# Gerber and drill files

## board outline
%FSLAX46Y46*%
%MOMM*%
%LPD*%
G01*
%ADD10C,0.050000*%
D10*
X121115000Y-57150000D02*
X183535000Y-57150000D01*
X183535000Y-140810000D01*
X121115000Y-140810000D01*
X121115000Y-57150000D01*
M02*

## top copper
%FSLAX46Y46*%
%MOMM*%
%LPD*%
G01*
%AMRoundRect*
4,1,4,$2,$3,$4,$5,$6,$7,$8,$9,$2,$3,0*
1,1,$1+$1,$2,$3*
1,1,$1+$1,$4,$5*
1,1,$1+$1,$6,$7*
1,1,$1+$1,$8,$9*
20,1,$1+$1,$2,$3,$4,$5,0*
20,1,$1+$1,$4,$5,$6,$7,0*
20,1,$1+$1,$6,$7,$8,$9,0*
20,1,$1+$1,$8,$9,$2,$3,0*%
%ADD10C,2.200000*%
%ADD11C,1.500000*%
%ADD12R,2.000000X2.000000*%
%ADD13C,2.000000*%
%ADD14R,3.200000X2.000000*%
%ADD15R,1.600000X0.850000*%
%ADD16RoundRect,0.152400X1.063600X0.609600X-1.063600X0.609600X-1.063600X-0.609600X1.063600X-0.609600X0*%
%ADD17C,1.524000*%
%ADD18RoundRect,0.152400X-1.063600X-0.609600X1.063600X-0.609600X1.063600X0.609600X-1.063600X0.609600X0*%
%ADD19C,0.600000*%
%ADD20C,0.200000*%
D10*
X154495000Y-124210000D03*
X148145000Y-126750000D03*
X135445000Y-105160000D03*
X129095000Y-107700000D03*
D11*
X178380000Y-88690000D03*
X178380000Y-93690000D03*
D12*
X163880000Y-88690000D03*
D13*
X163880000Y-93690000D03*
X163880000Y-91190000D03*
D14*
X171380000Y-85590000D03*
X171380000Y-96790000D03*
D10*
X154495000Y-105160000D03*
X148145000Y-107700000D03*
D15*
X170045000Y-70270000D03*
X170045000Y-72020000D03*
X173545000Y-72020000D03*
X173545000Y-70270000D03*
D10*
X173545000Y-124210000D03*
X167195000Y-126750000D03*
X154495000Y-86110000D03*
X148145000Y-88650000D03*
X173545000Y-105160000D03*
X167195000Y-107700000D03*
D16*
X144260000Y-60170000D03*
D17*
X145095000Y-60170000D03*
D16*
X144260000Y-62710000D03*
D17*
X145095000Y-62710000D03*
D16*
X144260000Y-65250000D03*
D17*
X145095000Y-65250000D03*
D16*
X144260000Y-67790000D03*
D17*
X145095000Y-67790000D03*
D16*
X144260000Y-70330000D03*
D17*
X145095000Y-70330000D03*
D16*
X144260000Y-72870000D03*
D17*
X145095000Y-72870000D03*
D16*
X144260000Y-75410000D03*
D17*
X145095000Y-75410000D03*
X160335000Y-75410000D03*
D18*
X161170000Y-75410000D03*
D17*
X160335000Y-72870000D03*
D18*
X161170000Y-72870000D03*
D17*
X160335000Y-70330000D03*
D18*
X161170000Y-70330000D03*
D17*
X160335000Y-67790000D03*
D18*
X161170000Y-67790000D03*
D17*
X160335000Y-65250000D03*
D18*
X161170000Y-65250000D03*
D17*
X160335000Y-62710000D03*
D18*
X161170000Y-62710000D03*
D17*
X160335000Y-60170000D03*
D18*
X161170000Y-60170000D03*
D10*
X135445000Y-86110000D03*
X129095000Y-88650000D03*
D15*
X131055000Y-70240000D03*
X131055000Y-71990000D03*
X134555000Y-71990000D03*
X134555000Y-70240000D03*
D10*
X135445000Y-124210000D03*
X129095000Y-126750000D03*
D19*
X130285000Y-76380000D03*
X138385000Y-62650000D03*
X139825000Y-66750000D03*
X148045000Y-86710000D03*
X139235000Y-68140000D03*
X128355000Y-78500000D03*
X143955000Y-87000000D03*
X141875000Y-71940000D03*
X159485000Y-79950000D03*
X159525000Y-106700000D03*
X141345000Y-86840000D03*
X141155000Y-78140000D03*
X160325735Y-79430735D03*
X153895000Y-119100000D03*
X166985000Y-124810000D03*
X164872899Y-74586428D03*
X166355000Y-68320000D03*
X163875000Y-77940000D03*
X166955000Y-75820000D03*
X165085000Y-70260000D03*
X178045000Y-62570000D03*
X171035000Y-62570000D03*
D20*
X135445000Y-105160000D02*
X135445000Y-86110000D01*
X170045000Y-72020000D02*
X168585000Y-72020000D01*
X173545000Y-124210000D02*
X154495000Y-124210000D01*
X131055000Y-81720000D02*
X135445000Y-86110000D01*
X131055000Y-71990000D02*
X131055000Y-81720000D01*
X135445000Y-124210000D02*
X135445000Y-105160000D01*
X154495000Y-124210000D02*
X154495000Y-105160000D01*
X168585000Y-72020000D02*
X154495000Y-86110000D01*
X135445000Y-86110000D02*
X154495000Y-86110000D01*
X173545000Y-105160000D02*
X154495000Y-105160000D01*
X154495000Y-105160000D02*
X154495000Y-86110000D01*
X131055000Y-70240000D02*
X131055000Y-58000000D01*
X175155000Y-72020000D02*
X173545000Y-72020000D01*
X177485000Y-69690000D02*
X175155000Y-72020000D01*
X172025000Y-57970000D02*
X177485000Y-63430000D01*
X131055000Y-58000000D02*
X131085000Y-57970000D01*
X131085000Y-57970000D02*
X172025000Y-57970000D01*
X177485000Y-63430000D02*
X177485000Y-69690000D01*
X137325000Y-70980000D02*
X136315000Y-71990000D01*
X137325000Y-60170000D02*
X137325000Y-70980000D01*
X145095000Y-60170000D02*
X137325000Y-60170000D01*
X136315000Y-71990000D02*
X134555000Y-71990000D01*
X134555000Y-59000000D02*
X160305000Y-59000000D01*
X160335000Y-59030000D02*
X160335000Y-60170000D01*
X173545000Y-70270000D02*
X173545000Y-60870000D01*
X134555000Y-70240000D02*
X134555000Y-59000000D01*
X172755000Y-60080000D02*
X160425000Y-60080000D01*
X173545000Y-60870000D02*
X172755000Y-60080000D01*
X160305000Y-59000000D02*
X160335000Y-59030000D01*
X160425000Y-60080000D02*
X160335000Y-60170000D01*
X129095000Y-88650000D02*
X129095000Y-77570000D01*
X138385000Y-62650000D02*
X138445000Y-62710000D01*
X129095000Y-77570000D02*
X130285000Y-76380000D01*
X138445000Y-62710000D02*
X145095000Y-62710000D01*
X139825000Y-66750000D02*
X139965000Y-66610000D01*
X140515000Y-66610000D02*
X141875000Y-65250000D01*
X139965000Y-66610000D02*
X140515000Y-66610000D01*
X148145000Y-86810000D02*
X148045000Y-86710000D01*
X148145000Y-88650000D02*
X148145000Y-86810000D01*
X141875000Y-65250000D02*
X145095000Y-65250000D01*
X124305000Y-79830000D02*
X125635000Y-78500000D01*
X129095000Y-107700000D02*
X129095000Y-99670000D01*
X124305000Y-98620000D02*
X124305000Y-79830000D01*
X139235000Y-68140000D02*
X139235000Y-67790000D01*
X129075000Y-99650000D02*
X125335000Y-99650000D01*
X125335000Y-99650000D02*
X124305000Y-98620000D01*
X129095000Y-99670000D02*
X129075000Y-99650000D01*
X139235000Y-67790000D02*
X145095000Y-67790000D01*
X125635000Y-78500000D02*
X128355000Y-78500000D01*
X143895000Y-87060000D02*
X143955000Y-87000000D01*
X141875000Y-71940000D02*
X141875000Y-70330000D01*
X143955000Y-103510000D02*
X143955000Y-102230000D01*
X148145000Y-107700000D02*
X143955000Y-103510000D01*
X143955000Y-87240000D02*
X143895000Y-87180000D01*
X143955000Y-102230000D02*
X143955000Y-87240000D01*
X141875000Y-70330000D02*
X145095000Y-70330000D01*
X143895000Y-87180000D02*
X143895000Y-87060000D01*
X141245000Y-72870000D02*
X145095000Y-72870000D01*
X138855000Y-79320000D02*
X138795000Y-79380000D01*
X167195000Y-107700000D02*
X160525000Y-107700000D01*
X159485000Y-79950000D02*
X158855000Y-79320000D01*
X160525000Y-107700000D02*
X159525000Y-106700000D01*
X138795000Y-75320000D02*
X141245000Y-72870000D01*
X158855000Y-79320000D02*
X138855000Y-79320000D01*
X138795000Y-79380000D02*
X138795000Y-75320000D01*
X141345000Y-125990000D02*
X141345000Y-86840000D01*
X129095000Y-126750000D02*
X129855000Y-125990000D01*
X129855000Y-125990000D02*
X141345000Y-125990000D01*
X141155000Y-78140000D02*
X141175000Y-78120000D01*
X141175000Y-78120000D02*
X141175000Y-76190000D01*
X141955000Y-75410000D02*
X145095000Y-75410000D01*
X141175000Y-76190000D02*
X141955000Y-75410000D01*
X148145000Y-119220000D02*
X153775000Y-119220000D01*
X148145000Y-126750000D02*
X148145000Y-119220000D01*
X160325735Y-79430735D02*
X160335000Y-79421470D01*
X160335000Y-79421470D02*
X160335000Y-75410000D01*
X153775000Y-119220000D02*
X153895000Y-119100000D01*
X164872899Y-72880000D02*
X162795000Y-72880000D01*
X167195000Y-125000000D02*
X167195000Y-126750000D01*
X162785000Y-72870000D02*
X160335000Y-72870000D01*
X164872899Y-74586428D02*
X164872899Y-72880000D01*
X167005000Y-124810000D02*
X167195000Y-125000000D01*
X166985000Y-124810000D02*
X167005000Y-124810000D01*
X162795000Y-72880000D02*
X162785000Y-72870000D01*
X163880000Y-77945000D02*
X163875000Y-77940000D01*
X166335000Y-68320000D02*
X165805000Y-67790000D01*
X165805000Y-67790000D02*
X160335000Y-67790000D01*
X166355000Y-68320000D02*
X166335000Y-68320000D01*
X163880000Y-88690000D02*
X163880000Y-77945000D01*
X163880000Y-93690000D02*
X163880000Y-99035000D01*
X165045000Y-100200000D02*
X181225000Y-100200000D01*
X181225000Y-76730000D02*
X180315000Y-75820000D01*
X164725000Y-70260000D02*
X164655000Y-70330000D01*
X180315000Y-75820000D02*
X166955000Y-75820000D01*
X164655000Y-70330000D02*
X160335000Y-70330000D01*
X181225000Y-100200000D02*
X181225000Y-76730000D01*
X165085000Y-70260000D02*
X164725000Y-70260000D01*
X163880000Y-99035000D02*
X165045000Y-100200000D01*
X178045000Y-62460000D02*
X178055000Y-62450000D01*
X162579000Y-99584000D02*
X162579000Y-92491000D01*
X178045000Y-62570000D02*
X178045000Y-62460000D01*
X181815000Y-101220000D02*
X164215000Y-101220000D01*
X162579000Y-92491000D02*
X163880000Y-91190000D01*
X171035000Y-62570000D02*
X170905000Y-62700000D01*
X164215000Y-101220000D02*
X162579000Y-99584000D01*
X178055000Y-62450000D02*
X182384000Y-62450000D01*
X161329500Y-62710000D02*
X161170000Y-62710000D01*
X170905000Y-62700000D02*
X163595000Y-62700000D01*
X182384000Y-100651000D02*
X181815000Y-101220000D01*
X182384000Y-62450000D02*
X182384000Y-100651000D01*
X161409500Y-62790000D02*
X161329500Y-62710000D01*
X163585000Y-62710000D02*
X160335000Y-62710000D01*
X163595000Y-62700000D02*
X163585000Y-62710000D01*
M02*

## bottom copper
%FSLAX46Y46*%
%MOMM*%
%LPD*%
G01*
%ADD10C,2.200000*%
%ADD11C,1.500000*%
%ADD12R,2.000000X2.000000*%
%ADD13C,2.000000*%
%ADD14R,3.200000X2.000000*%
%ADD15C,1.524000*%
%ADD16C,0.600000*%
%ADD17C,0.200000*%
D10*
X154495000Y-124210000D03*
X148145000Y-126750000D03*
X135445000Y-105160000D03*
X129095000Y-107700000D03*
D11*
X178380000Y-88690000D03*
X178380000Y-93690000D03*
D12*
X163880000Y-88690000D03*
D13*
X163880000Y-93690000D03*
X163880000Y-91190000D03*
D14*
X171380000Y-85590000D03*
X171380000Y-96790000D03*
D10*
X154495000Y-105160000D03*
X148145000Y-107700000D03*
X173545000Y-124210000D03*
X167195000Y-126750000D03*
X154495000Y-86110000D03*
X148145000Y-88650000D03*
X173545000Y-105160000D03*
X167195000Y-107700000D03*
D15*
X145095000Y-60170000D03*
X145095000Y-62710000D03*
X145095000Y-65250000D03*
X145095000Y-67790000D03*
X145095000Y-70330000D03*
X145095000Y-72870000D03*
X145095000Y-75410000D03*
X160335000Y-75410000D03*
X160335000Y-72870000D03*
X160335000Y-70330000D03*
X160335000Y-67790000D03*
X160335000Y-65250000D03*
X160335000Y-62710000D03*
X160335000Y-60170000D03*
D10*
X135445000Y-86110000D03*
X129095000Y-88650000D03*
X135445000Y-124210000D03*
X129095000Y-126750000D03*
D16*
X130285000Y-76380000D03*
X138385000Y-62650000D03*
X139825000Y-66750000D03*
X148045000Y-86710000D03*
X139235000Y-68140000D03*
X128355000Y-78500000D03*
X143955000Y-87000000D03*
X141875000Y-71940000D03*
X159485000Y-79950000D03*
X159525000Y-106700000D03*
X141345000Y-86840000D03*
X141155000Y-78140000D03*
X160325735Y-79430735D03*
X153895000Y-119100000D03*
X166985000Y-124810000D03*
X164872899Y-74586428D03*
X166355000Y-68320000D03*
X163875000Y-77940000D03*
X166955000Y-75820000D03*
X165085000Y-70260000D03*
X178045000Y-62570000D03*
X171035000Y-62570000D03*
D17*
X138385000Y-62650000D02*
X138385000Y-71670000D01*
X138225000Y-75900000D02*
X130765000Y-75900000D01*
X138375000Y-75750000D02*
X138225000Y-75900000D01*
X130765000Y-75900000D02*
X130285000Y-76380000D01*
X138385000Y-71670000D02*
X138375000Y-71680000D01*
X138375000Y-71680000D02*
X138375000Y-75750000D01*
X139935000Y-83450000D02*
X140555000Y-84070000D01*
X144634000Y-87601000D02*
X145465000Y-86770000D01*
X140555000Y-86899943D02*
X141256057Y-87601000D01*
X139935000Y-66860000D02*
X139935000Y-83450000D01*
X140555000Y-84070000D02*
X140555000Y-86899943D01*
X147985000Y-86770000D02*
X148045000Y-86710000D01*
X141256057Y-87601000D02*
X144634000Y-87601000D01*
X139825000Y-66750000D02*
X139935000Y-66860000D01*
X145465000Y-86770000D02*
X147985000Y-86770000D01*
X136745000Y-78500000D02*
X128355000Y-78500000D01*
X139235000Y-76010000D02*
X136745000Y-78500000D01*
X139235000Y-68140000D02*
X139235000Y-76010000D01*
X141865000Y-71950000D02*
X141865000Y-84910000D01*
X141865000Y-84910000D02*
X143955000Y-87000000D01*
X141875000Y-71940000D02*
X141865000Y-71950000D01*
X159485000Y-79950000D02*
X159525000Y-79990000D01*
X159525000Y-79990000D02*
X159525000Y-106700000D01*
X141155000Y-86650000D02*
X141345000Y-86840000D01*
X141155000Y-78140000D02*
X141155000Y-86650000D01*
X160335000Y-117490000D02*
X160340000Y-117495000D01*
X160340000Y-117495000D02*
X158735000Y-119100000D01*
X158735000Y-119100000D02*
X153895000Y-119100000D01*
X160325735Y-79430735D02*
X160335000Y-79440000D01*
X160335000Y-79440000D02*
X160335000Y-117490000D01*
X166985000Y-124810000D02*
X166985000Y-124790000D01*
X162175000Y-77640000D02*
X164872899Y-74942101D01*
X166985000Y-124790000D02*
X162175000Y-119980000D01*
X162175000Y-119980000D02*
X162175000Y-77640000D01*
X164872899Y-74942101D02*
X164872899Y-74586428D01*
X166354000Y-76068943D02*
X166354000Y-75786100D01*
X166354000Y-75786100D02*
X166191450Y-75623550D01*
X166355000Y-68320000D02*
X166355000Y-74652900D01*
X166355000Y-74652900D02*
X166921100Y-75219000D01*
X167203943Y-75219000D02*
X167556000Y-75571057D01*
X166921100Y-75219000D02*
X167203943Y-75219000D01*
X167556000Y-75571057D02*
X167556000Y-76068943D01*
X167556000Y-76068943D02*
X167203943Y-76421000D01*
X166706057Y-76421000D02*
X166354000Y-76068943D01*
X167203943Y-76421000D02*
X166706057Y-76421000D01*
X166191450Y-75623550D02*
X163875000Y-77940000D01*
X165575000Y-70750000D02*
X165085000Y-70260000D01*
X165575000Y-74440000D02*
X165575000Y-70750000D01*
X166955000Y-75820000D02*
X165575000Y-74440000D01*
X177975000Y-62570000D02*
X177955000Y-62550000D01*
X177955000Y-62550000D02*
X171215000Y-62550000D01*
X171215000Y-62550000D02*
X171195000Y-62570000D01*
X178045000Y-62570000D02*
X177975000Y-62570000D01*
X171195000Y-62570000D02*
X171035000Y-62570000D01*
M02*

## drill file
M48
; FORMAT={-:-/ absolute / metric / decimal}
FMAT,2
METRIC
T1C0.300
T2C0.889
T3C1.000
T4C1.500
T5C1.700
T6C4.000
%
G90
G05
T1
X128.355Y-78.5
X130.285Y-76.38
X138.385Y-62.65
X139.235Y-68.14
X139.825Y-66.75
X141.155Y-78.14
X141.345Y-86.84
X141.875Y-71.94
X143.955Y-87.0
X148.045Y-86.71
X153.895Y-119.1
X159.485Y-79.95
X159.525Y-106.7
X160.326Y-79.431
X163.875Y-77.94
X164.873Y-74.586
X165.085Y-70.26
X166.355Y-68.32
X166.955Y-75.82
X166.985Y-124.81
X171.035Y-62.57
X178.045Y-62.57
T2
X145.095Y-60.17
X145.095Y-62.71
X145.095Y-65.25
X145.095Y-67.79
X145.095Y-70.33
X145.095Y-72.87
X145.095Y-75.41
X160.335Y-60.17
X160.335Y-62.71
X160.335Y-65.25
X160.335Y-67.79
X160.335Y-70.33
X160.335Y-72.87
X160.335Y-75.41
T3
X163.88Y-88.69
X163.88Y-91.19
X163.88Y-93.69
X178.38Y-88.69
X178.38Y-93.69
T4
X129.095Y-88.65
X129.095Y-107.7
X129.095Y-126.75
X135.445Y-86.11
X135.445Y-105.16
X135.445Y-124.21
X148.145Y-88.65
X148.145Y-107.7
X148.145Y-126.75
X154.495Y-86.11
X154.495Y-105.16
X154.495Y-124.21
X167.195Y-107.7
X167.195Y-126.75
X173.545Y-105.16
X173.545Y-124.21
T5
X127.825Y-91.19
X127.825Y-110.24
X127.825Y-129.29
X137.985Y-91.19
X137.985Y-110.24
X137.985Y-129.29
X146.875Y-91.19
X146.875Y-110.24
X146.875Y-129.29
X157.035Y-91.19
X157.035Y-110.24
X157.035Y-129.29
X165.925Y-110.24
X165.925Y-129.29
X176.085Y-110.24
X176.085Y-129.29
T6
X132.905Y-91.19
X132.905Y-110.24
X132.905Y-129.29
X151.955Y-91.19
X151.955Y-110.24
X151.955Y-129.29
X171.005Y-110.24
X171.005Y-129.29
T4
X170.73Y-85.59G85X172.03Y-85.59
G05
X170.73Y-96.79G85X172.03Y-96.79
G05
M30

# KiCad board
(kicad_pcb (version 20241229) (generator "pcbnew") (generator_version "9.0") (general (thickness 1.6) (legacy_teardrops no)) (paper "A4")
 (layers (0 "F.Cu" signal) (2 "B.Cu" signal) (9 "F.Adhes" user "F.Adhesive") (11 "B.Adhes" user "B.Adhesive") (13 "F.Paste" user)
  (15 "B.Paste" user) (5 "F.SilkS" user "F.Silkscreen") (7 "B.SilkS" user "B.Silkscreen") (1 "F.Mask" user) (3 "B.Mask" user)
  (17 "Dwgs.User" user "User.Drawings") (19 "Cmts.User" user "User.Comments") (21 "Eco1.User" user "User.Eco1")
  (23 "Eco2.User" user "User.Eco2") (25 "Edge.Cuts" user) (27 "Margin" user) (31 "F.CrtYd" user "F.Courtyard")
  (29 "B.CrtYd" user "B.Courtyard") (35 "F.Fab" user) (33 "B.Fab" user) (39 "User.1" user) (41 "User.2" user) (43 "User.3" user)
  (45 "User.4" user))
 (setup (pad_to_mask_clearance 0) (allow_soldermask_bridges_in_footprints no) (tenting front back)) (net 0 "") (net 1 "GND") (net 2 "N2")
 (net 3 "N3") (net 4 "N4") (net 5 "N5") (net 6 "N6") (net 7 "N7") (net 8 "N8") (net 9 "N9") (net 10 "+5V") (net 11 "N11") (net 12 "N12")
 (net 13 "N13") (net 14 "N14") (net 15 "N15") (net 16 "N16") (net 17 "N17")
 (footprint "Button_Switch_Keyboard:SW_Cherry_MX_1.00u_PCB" (layer "F.Cu") (at 154.495 124.21)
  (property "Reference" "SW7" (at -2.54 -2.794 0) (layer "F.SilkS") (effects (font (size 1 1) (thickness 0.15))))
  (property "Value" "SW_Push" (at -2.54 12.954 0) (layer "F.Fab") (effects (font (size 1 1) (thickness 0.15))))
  (pad "" np_thru_hole circle (at -7.62 5.08) (size 1.7 1.7) (drill 1.7) (layers "*.Cu" "*.Mask"))
  (pad "" np_thru_hole circle (at -2.54 5.08) (size 4 4) (drill 4) (layers "*.Cu" "*.Mask"))
  (pad "" np_thru_hole circle (at 2.54 5.08) (size 1.7 1.7) (drill 1.7) (layers "*.Cu" "*.Mask"))
  (pad "1" thru_hole circle (at 0 0) (size 2.2 2.2) (drill 1.5) (layers "*.Cu" "*.Mask") (remove_unused_layers no) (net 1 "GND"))
  (pad "2" thru_hole circle (at -6.35 2.54) (size 2.2 2.2) (drill 1.5) (layers "*.Cu" "*.Mask") (remove_unused_layers no) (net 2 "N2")))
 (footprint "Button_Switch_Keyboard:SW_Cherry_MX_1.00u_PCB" (layer "F.Cu") (at 135.445 105.16)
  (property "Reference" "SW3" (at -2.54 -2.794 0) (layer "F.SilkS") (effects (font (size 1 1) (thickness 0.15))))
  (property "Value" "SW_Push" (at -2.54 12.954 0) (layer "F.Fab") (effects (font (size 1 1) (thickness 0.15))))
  (pad "" np_thru_hole circle (at -7.62 5.08) (size 1.7 1.7) (drill 1.7) (layers "*.Cu" "*.Mask"))
  (pad "" np_thru_hole circle (at -2.54 5.08) (size 4 4) (drill 4) (layers "*.Cu" "*.Mask"))
  (pad "" np_thru_hole circle (at 2.54 5.08) (size 1.7 1.7) (drill 1.7) (layers "*.Cu" "*.Mask"))
  (pad "1" thru_hole circle (at 0 0) (size 2.2 2.2) (drill 1.5) (layers "*.Cu" "*.Mask") (remove_unused_layers no) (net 1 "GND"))
  (pad "2" thru_hole circle (at -6.35 2.54) (size 2.2 2.2) (drill 1.5) (layers "*.Cu" "*.Mask") (remove_unused_layers no) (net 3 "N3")))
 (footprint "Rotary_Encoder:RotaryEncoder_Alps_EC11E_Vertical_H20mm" (layer "F.Cu") (at 163.88 88.69)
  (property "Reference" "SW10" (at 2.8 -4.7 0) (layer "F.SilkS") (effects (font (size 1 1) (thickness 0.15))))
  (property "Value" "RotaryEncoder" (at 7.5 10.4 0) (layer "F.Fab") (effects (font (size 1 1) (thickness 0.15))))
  (pad "" thru_hole circle (at 14.5 0) (size 1.5 1.5) (drill 1) (layers "*.Cu" "*.Mask") (remove_unused_layers no))
  (pad "" thru_hole circle (at 14.5 5) (size 1.5 1.5) (drill 1) (layers "*.Cu" "*.Mask") (remove_unused_layers no))
  (pad "A" thru_hole rect (at 0 0) (size 2 2) (drill 1) (layers "*.Cu" "*.Mask") (remove_unused_layers no) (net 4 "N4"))
  (pad "B" thru_hole circle (at 0 5) (size 2 2) (drill 1) (layers "*.Cu" "*.Mask") (remove_unused_layers no) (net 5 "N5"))
  (pad "C" thru_hole circle (at 0 2.5) (size 2 2) (drill 1) (layers "*.Cu" "*.Mask") (remove_unused_layers no) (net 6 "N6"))
  (pad "MP" thru_hole rect (at 7.5 -3.1) (size 3.2 2) (drill oval 2.8 1.5) (layers "*.Cu" "*.Mask") (remove_unused_layers no))
  (pad "MP" thru_hole rect (at 7.5 8.1) (size 3.2 2) (drill oval 2.8 1.5) (layers "*.Cu" "*.Mask") (remove_unused_layers no)))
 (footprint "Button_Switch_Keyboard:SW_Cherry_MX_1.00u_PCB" (layer "F.Cu") (at 154.495 105.16)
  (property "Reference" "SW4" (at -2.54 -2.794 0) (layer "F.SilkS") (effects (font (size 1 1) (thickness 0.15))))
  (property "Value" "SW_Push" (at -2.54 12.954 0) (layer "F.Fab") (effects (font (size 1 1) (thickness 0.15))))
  (pad "" np_thru_hole circle (at -7.62 5.08) (size 1.7 1.7) (drill 1.7) (layers "*.Cu" "*.Mask"))
  (pad "" np_thru_hole circle (at -2.54 5.08) (size 4 4) (drill 4) (layers "*.Cu" "*.Mask"))
  (pad "" np_thru_hole circle (at 2.54 5.08) (size 1.7 1.7) (drill 1.7) (layers "*.Cu" "*.Mask"))
  (pad "1" thru_hole circle (at 0 0) (size 2.2 2.2) (drill 1.5) (layers "*.Cu" "*.Mask") (remove_unused_layers no) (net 1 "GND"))
  (pad "2" thru_hole circle (at -6.35 2.54) (size 2.2 2.2) (drill 1.5) (layers "*.Cu" "*.Mask") (remove_unused_layers no) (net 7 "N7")))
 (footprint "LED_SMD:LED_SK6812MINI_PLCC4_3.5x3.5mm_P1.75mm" (layer "F.Cu") (at 171.795 71.145)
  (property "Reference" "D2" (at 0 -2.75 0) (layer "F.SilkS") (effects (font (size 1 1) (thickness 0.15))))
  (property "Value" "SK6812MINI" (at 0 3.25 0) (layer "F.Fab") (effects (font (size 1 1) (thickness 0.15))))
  (pad "1" smd rect (at -1.75 -0.875) (size 1.6 0.85) (layers "F.Cu" "F.Mask" "F.Paste") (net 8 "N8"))
  (pad "2" smd rect (at -1.75 0.875) (size 1.6 0.85) (layers "F.Cu" "F.Mask" "F.Paste") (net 1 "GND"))
  (pad "3" smd rect (at 1.75 0.875) (size 1.6 0.85) (layers "F.Cu" "F.Mask" "F.Paste") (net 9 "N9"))
  (pad "4" smd rect (at 1.75 -0.875) (size 1.6 0.85) (layers "F.Cu" "F.Mask" "F.Paste") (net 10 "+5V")))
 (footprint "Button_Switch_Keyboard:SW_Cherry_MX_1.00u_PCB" (layer "F.Cu") (at 173.545 124.21)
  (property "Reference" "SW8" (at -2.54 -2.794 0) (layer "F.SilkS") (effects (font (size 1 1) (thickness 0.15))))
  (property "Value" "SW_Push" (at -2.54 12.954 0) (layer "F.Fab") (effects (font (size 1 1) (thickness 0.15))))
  (pad "" np_thru_hole circle (at -7.62 5.08) (size 1.7 1.7) (drill 1.7) (layers "*.Cu" "*.Mask"))
  (pad "" np_thru_hole circle (at -2.54 5.08) (size 4 4) (drill 4) (layers "*.Cu" "*.Mask"))
  (pad "" np_thru_hole circle (at 2.54 5.08) (size 1.7 1.7) (drill 1.7) (layers "*.Cu" "*.Mask"))
  (pad "1" thru_hole circle (at 0 0) (size 2.2 2.2) (drill 1.5) (layers "*.Cu" "*.Mask") (remove_unused_layers no) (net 1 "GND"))
  (pad "2" thru_hole circle (at -6.35 2.54) (size 2.2 2.2) (drill 1.5) (layers "*.Cu" "*.Mask") (remove_unused_layers no) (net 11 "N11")))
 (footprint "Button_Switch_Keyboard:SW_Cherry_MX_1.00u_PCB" (layer "F.Cu") (at 154.495 86.11)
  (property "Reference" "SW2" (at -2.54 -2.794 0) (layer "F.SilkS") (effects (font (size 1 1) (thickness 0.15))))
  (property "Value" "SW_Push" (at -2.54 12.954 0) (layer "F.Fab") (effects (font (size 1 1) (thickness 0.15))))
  (pad "" np_thru_hole circle (at -7.62 5.08) (size 1.7 1.7) (drill 1.7) (layers "*.Cu" "*.Mask"))
  (pad "" np_thru_hole circle (at -2.54 5.08) (size 4 4) (drill 4) (layers "*.Cu" "*.Mask"))
  (pad "" np_thru_hole circle (at 2.54 5.08) (size 1.7 1.7) (drill 1.7) (layers "*.Cu" "*.Mask"))
  (pad "1" thru_hole circle (at 0 0) (size 2.2 2.2) (drill 1.5) (layers "*.Cu" "*.Mask") (remove_unused_layers no) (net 1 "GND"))
  (pad "2" thru_hole circle (at -6.35 2.54) (size 2.2 2.2) (drill 1.5) (layers "*.Cu" "*.Mask") (remove_unused_layers no) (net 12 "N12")))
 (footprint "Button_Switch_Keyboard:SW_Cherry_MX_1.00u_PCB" (layer "F.Cu") (at 173.545 105.16)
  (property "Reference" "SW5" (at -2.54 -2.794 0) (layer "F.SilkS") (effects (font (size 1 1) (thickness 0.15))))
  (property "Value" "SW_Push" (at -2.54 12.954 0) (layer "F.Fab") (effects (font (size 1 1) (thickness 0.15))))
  (pad "" np_thru_hole circle (at -7.62 5.08) (size 1.7 1.7) (drill 1.7) (layers "*.Cu" "*.Mask"))
  (pad "" np_thru_hole circle (at -2.54 5.08) (size 4 4) (drill 4) (layers "*.Cu" "*.Mask"))
  (pad "" np_thru_hole circle (at 2.54 5.08) (size 1.7 1.7) (drill 1.7) (layers "*.Cu" "*.Mask"))
  (pad "1" thru_hole circle (at 0 0) (size 2.2 2.2) (drill 1.5) (layers "*.Cu" "*.Mask") (remove_unused_layers no) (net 1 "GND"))
  (pad "2" thru_hole circle (at -6.35 2.54) (size 2.2 2.2) (drill 1.5) (layers "*.Cu" "*.Mask") (remove_unused_layers no) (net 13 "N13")))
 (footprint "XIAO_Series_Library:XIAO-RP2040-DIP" (layer "F.Cu") (at 152.715 67.79)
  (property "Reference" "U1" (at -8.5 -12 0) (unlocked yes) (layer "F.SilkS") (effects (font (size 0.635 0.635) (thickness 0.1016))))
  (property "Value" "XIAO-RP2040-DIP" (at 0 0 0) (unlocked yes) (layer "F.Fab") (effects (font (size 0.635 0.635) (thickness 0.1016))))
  (pad "1" smd roundrect (at -8.455 -7.62 180) (size 2.432 1.524) (layers "F.Cu" "F.Mask") (roundrect_rratio 0.1) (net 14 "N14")
   (thermal_bridge_angle 45))
  (pad "1" thru_hole circle (at -7.62 -7.62 180) (size 1.524 1.524) (drill 0.889) (layers "*.Cu" "*.Mask") (remove_unused_layers no)
   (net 14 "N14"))
  (pad "2" smd roundrect (at -8.455 -5.08 180) (size 2.432 1.524) (layers "F.Cu" "F.Mask") (roundrect_rratio 0.1) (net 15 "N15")
   (thermal_bridge_angle 45))
  (pad "2" thru_hole circle (at -7.62 -5.08 180) (size 1.524 1.524) (drill 0.889) (layers "*.Cu" "*.Mask") (remove_unused_layers no)
   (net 15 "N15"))
  (pad "3" smd roundrect (at -8.455 -2.54 180) (size 2.432 1.524) (layers "F.Cu" "F.Mask") (roundrect_rratio 0.1) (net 12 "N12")
   (thermal_bridge_angle 45))
  (pad "3" thru_hole circle (at -7.62 -2.54 180) (size 1.524 1.524) (drill 0.889) (layers "*.Cu" "*.Mask") (remove_unused_layers no)
   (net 12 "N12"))
  (pad "4" smd roundrect (at -8.455 0 180) (size 2.432 1.524) (layers "F.Cu" "F.Mask") (roundrect_rratio 0.1) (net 3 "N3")
   (thermal_bridge_angle 45))
  (pad "4" thru_hole circle (at -7.62 0 180) (size 1.524 1.524) (drill 0.889) (layers "*.Cu" "*.Mask") (remove_unused_layers no)
   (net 3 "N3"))
  (pad "5" smd roundrect (at -8.455 2.54 180) (size 2.432 1.524) (layers "F.Cu" "F.Mask") (roundrect_rratio 0.1) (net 7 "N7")
   (thermal_bridge_angle 45))
  (pad "5" thru_hole circle (at -7.62 2.54 180) (size 1.524 1.524) (drill 0.889) (layers "*.Cu" "*.Mask") (remove_unused_layers no)
   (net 7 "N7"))
  (pad "6" smd roundrect (at -8.455 5.08 180) (size 2.432 1.524) (layers "F.Cu" "F.Mask") (roundrect_rratio 0.1) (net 13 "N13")
   (thermal_bridge_angle 45))
  (pad "6" thru_hole circle (at -7.62 5.08 180) (size 1.524 1.524) (drill 0.889) (layers "*.Cu" "*.Mask") (remove_unused_layers no)
   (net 13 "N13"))
  (pad "7" smd roundrect (at -8.455 7.62 180) (size 2.432 1.524) (layers "F.Cu" "F.Mask") (roundrect_rratio 0.1) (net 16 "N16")
   (thermal_bridge_angle 45))
  (pad "7" thru_hole circle (at -7.62 7.62 180) (size 1.524 1.524) (drill 0.889) (layers "*.Cu" "*.Mask") (remove_unused_layers no)
   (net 16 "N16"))
  (pad "8" thru_hole circle (at 7.62 7.62) (size 1.524 1.524) (drill 0.889) (layers "*.Cu" "*.Mask") (remove_unused_layers no) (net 2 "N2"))
  (pad "8" smd roundrect (at 8.455 7.62) (size 2.432 1.524) (layers "F.Cu" "F.Mask") (roundrect_rratio 0.1) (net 2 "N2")
   (thermal_bridge_angle 45))
  (pad "9" thru_hole circle (at 7.62 5.08) (size 1.524 1.524) (drill 0.889) (layers "*.Cu" "*.Mask") (remove_unused_layers no)
   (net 11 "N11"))
  (pad "9" smd roundrect (at 8.455 5.08) (size 2.432 1.524) (layers "F.Cu" "F.Mask") (roundrect_rratio 0.1) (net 11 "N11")
   (thermal_bridge_angle 45))
  (pad "10" thru_hole circle (at 7.62 2.54) (size 1.524 1.524) (drill 0.889) (layers "*.Cu" "*.Mask") (remove_unused_layers no) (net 5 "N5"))
  (pad "10" smd roundrect (at 8.455 2.54) (size 2.432 1.524) (layers "F.Cu" "F.Mask") (roundrect_rratio 0.1) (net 5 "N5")
   (thermal_bridge_angle 45))
  (pad "11" thru_hole circle (at 7.62 0) (size 1.524 1.524) (drill 0.889) (layers "*.Cu" "*.Mask") (remove_unused_layers no) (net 4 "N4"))
  (pad "11" smd roundrect (at 8.455 0) (size 2.432 1.524) (layers "F.Cu" "F.Mask") (roundrect_rratio 0.1) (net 4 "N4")
   (thermal_bridge_angle 45))
  (pad "12" thru_hole circle (at 7.62 -2.54) (size 1.524 1.524) (drill 0.889) (layers "*.Cu" "*.Mask") (remove_unused_layers no)
   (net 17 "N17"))
  (pad "12" smd roundrect (at 8.455 -2.54) (size 2.432 1.524) (layers "F.Cu" "F.Mask") (roundrect_rratio 0.1) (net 17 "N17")
   (thermal_bridge_angle 45))
  (pad "13" thru_hole circle (at 7.62 -5.08) (size 1.524 1.524) (drill 0.889) (layers "*.Cu" "*.Mask") (remove_unused_layers no)
   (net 6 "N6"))
  (pad "13" smd roundrect (at 8.455 -5.08) (size 2.432 1.524) (layers "F.Cu" "F.Mask") (roundrect_rratio 0.1) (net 6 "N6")
   (thermal_bridge_angle 45))
  (pad "14" thru_hole circle (at 7.62 -7.62) (size 1.524 1.524) (drill 0.889) (layers "*.Cu" "*.Mask") (remove_unused_layers no)
   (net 10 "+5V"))
  (pad "14" smd roundrect (at 8.455 -7.62) (size 2.432 1.524) (layers "F.Cu" "F.Mask") (roundrect_rratio 0.1) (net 10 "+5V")
   (thermal_bridge_angle 45)))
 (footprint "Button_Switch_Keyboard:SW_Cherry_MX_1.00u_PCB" (layer "F.Cu") (at 135.445 86.11)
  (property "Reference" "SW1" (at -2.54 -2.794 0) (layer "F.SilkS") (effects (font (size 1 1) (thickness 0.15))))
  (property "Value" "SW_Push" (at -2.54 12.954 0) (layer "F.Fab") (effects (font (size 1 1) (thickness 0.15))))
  (pad "" np_thru_hole circle (at -7.62 5.08) (size 1.7 1.7) (drill 1.7) (layers "*.Cu" "*.Mask"))
  (pad "" np_thru_hole circle (at -2.54 5.08) (size 4 4) (drill 4) (layers "*.Cu" "*.Mask"))
  (pad "" np_thru_hole circle (at 2.54 5.08) (size 1.7 1.7) (drill 1.7) (layers "*.Cu" "*.Mask"))
  (pad "1" thru_hole circle (at 0 0) (size 2.2 2.2) (drill 1.5) (layers "*.Cu" "*.Mask") (remove_unused_layers no) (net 1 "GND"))
  (pad "2" thru_hole circle (at -6.35 2.54) (size 2.2 2.2) (drill 1.5) (layers "*.Cu" "*.Mask") (remove_unused_layers no) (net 15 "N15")))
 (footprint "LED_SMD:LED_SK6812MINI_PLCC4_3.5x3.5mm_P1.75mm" (layer "F.Cu") (at 132.805 71.115)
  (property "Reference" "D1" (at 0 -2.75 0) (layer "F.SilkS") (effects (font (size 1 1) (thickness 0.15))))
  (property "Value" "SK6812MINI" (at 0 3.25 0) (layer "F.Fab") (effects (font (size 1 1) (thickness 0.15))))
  (pad "1" smd rect (at -1.75 -0.875) (size 1.6 0.85) (layers "F.Cu" "F.Mask" "F.Paste") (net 9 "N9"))
  (pad "2" smd rect (at -1.75 0.875) (size 1.6 0.85) (layers "F.Cu" "F.Mask" "F.Paste") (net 1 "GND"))
  (pad "3" smd rect (at 1.75 0.875) (size 1.6 0.85) (layers "F.Cu" "F.Mask" "F.Paste") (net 14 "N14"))
  (pad "4" smd rect (at 1.75 -0.875) (size 1.6 0.85) (layers "F.Cu" "F.Mask" "F.Paste") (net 10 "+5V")))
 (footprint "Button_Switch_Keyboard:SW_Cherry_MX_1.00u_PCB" (layer "F.Cu") (at 135.445 124.21)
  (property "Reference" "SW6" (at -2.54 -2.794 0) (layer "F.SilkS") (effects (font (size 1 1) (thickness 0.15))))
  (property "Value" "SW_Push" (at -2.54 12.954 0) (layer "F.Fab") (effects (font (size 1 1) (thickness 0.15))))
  (pad "" np_thru_hole circle (at -7.62 5.08) (size 1.7 1.7) (drill 1.7) (layers "*.Cu" "*.Mask"))
  (pad "" np_thru_hole circle (at -2.54 5.08) (size 4 4) (drill 4) (layers "*.Cu" "*.Mask"))
  (pad "" np_thru_hole circle (at 2.54 5.08) (size 1.7 1.7) (drill 1.7) (layers "*.Cu" "*.Mask"))
  (pad "1" thru_hole circle (at 0 0) (size 2.2 2.2) (drill 1.5) (layers "*.Cu" "*.Mask") (remove_unused_layers no) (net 1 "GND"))
  (pad "2" thru_hole circle (at -6.35 2.54) (size 2.2 2.2) (drill 1.5) (layers "*.Cu" "*.Mask") (remove_unused_layers no) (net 16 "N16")))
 (gr_rect (start 121.115 57.15) (end 183.535 140.81) (stroke (width 0.05) (type default)) (fill no) (layer "Edge.Cuts"))
 (segment (start 135.445 105.16) (end 135.445 86.11) (width 0.2) (layer "F.Cu") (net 1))
 (segment (start 170.045 72.02) (end 168.585 72.02) (width 0.2) (layer "F.Cu") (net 1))
 (segment (start 173.545 124.21) (end 154.495 124.21) (width 0.2) (layer "F.Cu") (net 1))
 (segment (start 131.055 81.72) (end 135.445 86.11) (width 0.2) (layer "F.Cu") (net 1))
 (segment (start 131.055 71.99) (end 131.055 81.72) (width 0.2) (layer "F.Cu") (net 1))
 (segment (start 135.445 124.21) (end 135.445 105.16) (width 0.2) (layer "F.Cu") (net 1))
 (segment (start 154.495 124.21) (end 154.495 105.16) (width 0.2) (layer "F.Cu") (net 1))
 (segment (start 168.585 72.02) (end 154.495 86.11) (width 0.2) (layer "F.Cu") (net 1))
 (segment (start 135.445 86.11) (end 154.495 86.11) (width 0.2) (layer "F.Cu") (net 1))
 (segment (start 173.545 105.16) (end 154.495 105.16) (width 0.2) (layer "F.Cu") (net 1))
 (segment (start 154.495 105.16) (end 154.495 86.11) (width 0.2) (layer "F.Cu") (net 1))
 (segment (start 131.055 70.24) (end 131.055 58) (width 0.2) (layer "F.Cu") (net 9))
 (segment (start 175.155 72.02) (end 173.545 72.02) (width 0.2) (layer "F.Cu") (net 9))
 (segment (start 177.485 69.69) (end 175.155 72.02) (width 0.2) (layer "F.Cu") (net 9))
 (segment (start 172.025 57.97) (end 177.485 63.43) (width 0.2) (layer "F.Cu") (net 9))
 (segment (start 131.055 58) (end 131.085 57.97) (width 0.2) (layer "F.Cu") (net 9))
 (segment (start 131.085 57.97) (end 172.025 57.97) (width 0.2) (layer "F.Cu") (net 9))
 (segment (start 177.485 63.43) (end 177.485 69.69) (width 0.2) (layer "F.Cu") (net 9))
 (segment (start 137.325 70.98) (end 136.315 71.99) (width 0.2) (layer "F.Cu") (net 14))
 (segment (start 137.325 60.17) (end 137.325 70.98) (width 0.2) (layer "F.Cu") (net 14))
 (segment (start 145.095 60.17) (end 137.325 60.17) (width 0.2) (layer "F.Cu") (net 14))
 (segment (start 136.315 71.99) (end 134.555 71.99) (width 0.2) (layer "F.Cu") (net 14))
 (segment (start 134.555 59) (end 160.305 59) (width 0.2) (layer "F.Cu") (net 10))
 (segment (start 160.335 59.03) (end 160.335 60.17) (width 0.2) (layer "F.Cu") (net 10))
 (segment (start 173.545 70.27) (end 173.545 60.87) (width 0.2) (layer "F.Cu") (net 10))
 (segment (start 134.555 70.24) (end 134.555 59) (width 0.2) (layer "F.Cu") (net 10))
 (segment (start 172.755 60.08) (end 160.425 60.08) (width 0.2) (layer "F.Cu") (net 10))
 (segment (start 173.545 60.87) (end 172.755 60.08) (width 0.2) (layer "F.Cu") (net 10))
 (segment (start 160.305 59) (end 160.335 59.03) (width 0.2) (layer "F.Cu") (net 10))
 (segment (start 160.425 60.08) (end 160.335 60.17) (width 0.2) (layer "F.Cu") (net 10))
 (segment (start 129.095 88.65) (end 129.095 77.57) (width 0.2) (layer "F.Cu") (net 15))
 (segment (start 138.385 62.65) (end 138.445 62.71) (width 0.2) (layer "F.Cu") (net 15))
 (segment (start 129.095 77.57) (end 130.285 76.38) (width 0.2) (layer "F.Cu") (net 15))
 (segment (start 138.445 62.71) (end 145.095 62.71) (width 0.2) (layer "F.Cu") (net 15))
 (via (at 130.285 76.38) (size 0.6) (drill 0.3) (layers "F.Cu" "B.Cu") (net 15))
 (via (at 138.385 62.65) (size 0.6) (drill 0.3) (layers "F.Cu" "B.Cu") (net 15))
 (segment (start 138.385 62.65) (end 138.385 71.67) (width 0.2) (layer "B.Cu") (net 15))
 (segment (start 138.225 75.9) (end 130.765 75.9) (width 0.2) (layer "B.Cu") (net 15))
 (segment (start 138.375 75.75) (end 138.225 75.9) (width 0.2) (layer "B.Cu") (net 15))
 (segment (start 130.765 75.9) (end 130.285 76.38) (width 0.2) (layer "B.Cu") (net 15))
 (segment (start 138.385 71.67) (end 138.375 71.68) (width 0.2) (layer "B.Cu") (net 15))
 (segment (start 138.375 71.68) (end 138.375 75.75) (width 0.2) (layer "B.Cu") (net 15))
 (segment (start 139.825 66.75) (end 139.965 66.61) (width 0.2) (layer "F.Cu") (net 12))
 (segment (start 140.515 66.61) (end 141.875 65.25) (width 0.2) (layer "F.Cu") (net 12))
 (segment (start 139.965 66.61) (end 140.515 66.61) (width 0.2) (layer "F.Cu") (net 12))
 (segment (start 148.145 86.81) (end 148.045 86.71) (width 0.2) (layer "F.Cu") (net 12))
 (segment (start 148.145 88.65) (end 148.145 86.81) (width 0.2) (layer "F.Cu") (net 12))
 (segment (start 141.875 65.25) (end 145.095 65.25) (width 0.2) (layer "F.Cu") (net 12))
 (via (at 139.825 66.75) (size 0.6) (drill 0.3) (layers "F.Cu" "B.Cu") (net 12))
 (via (at 148.045 86.71) (size 0.6) (drill 0.3) (layers "F.Cu" "B.Cu") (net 12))
 (segment (start 139.935 83.45) (end 140.555 84.07) (width 0.2) (layer "B.Cu") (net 12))
 (segment (start 144.634 87.601) (end 145.465 86.77) (width 0.2) (layer "B.Cu") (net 12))
 (segment (start 140.555 86.899943) (end 141.256057 87.601) (width 0.2) (layer "B.Cu") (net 12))
 (segment (start 139.935 66.86) (end 139.935 83.45) (width 0.2) (layer "B.Cu") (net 12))
 (segment (start 140.555 84.07) (end 140.555 86.899943) (width 0.2) (layer "B.Cu") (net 12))
 (segment (start 147.985 86.77) (end 148.045 86.71) (width 0.2) (layer "B.Cu") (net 12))
 (segment (start 141.256057 87.601) (end 144.634 87.601) (width 0.2) (layer "B.Cu") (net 12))
 (segment (start 139.825 66.75) (end 139.935 66.86) (width 0.2) (layer "B.Cu") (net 12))
 (segment (start 145.465 86.77) (end 147.985 86.77) (width 0.2) (layer "B.Cu") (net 12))
 (segment (start 124.305 79.83) (end 125.635 78.5) (width 0.2) (layer "F.Cu") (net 3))
 (segment (start 129.095 107.7) (end 129.095 99.67) (width 0.2) (layer "F.Cu") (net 3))
 (segment (start 124.305 98.62) (end 124.305 79.83) (width 0.2) (layer "F.Cu") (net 3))
 (segment (start 139.235 68.14) (end 139.235 67.79) (width 0.2) (layer "F.Cu") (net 3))
 (segment (start 129.075 99.65) (end 125.335 99.65) (width 0.2) (layer "F.Cu") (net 3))
 (segment (start 125.335 99.65) (end 124.305 98.62) (width 0.2) (layer "F.Cu") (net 3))
 (segment (start 129.095 99.67) (end 129.075 99.65) (width 0.2) (layer "F.Cu") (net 3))
 (segment (start 139.235 67.79) (end 145.095 67.79) (width 0.2) (layer "F.Cu") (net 3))
 (segment (start 125.635 78.5) (end 128.355 78.5) (width 0.2) (layer "F.Cu") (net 3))
 (via (at 139.235 68.14) (size 0.6) (drill 0.3) (layers "F.Cu" "B.Cu") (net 3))
 (via (at 128.355 78.5) (size 0.6) (drill 0.3) (layers "F.Cu" "B.Cu") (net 3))
 (segment (start 136.745 78.5) (end 128.355 78.5) (width 0.2) (layer "B.Cu") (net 3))
 (segment (start 139.235 76.01) (end 136.745 78.5) (width 0.2) (layer "B.Cu") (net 3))
 (segment (start 139.235 68.14) (end 139.235 76.01) (width 0.2) (layer "B.Cu") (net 3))
 (segment (start 143.895 87.06) (end 143.955 87) (width 0.2) (layer "F.Cu") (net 7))
 (segment (start 141.875 71.94) (end 141.875 70.33) (width 0.2) (layer "F.Cu") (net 7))
 (segment (start 143.955 103.51) (end 143.955 102.23) (width 0.2) (layer "F.Cu") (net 7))
 (segment (start 148.145 107.7) (end 143.955 103.51) (width 0.2) (layer "F.Cu") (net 7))
 (segment (start 143.955 87.24) (end 143.895 87.18) (width 0.2) (layer "F.Cu") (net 7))
 (segment (start 143.955 102.23) (end 143.955 87.24) (width 0.2) (layer "F.Cu") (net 7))
 (segment (start 141.875 70.33) (end 145.095 70.33) (width 0.2) (layer "F.Cu") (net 7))
 (segment (start 143.895 87.18) (end 143.895 87.06) (width 0.2) (layer "F.Cu") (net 7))
 (via (at 143.955 87) (size 0.6) (drill 0.3) (layers "F.Cu" "B.Cu") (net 7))
 (via (at 141.875 71.94) (size 0.6) (drill 0.3) (layers "F.Cu" "B.Cu") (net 7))
 (segment (start 141.865 71.95) (end 141.865 84.91) (width 0.2) (layer "B.Cu") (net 7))
 (segment (start 141.865 84.91) (end 143.955 87) (width 0.2) (layer "B.Cu") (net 7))
 (segment (start 141.875 71.94) (end 141.865 71.95) (width 0.2) (layer "B.Cu") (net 7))
 (segment (start 141.245 72.87) (end 145.095 72.87) (width 0.2) (layer "F.Cu") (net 13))
 (segment (start 138.855 79.32) (end 138.795 79.38) (width 0.2) (layer "F.Cu") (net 13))
 (segment (start 167.195 107.7) (end 160.525 107.7) (width 0.2) (layer "F.Cu") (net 13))
 (segment (start 159.485 79.95) (end 158.855 79.32) (width 0.2) (layer "F.Cu") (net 13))
 (segment (start 160.525 107.7) (end 159.525 106.7) (width 0.2) (layer "F.Cu") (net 13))
 (segment (start 138.795 75.32) (end 141.245 72.87) (width 0.2) (layer "F.Cu") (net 13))
 (segment (start 158.855 79.32) (end 138.855 79.32) (width 0.2) (layer "F.Cu") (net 13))
 (segment (start 138.795 79.38) (end 138.795 75.32) (width 0.2) (layer "F.Cu") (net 13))
 (via (at 159.485 79.95) (size 0.6) (drill 0.3) (layers "F.Cu" "B.Cu") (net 13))
 (via (at 159.525 106.7) (size 0.6) (drill 0.3) (layers "F.Cu" "B.Cu") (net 13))
 (segment (start 159.485 79.95) (end 159.525 79.99) (width 0.2) (layer "B.Cu") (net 13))
 (segment (start 159.525 79.99) (end 159.525 106.7) (width 0.2) (layer "B.Cu") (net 13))
 (segment (start 141.345 125.99) (end 141.345 86.84) (width 0.2) (layer "F.Cu") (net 16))
 (segment (start 129.095 126.75) (end 129.855 125.99) (width 0.2) (layer "F.Cu") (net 16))
 (segment (start 129.855 125.99) (end 141.345 125.99) (width 0.2) (layer "F.Cu") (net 16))
 (segment (start 141.155 78.14) (end 141.175 78.12) (width 0.2) (layer "F.Cu") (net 16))
 (segment (start 141.175 78.12) (end 141.175 76.19) (width 0.2) (layer "F.Cu") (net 16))
 (segment (start 141.955 75.41) (end 145.095 75.41) (width 0.2) (layer "F.Cu") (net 16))
 (segment (start 141.175 76.19) (end 141.955 75.41) (width 0.2) (layer "F.Cu") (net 16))
 (via (at 141.345 86.84) (size 0.6) (drill 0.3) (layers "F.Cu" "B.Cu") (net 16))
 (via (at 141.155 78.14) (size 0.6) (drill 0.3) (layers "F.Cu" "B.Cu") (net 16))
 (segment (start 141.155 86.65) (end 141.345 86.84) (width 0.2) (layer "B.Cu") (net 16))
 (segment (start 141.155 78.14) (end 141.155 86.65) (width 0.2) (layer "B.Cu") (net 16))
 (segment (start 148.145 119.22) (end 153.775 119.22) (width 0.2) (layer "F.Cu") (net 2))
 (segment (start 148.145 126.75) (end 148.145 119.22) (width 0.2) (layer "F.Cu") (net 2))
 (segment (start 160.325735 79.430735) (end 160.335 79.42147) (width 0.2) (layer "F.Cu") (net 2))
 (segment (start 160.335 79.42147) (end 160.335 75.41) (width 0.2) (layer "F.Cu") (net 2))
 (segment (start 153.775 119.22) (end 153.895 119.1) (width 0.2) (layer "F.Cu") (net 2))
 (via (at 160.325735 79.430735) (size 0.6) (drill 0.3) (layers "F.Cu" "B.Cu") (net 2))
 (via (at 153.895 119.1) (size 0.6) (drill 0.3) (layers "F.Cu" "B.Cu") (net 2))
 (segment (start 160.335 117.49) (end 160.34 117.495) (width 0.2) (layer "B.Cu") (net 2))
 (segment (start 160.34 117.495) (end 158.735 119.1) (width 0.2) (layer "B.Cu") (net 2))
 (segment (start 158.735 119.1) (end 153.895 119.1) (width 0.2) (layer "B.Cu") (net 2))
 (segment (start 160.325735 79.430735) (end 160.335 79.44) (width 0.2) (layer "B.Cu") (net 2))
 (segment (start 160.335 79.44) (end 160.335 117.49) (width 0.2) (layer "B.Cu") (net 2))
 (segment (start 164.872899 72.88) (end 162.795 72.88) (width 0.2) (layer "F.Cu") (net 11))
 (segment (start 167.195 125) (end 167.195 126.75) (width 0.2) (layer "F.Cu") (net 11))
 (segment (start 162.785 72.87) (end 160.335 72.87) (width 0.2) (layer "F.Cu") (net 11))
 (segment (start 164.872899 74.586428) (end 164.872899 72.88) (width 0.2) (layer "F.Cu") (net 11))
 (segment (start 167.005 124.81) (end 167.195 125) (width 0.2) (layer "F.Cu") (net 11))
 (segment (start 166.985 124.81) (end 167.005 124.81) (width 0.2) (layer "F.Cu") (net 11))
 (segment (start 162.795 72.88) (end 162.785 72.87) (width 0.2) (layer "F.Cu") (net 11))
 (via (at 166.985 124.81) (size 0.6) (drill 0.3) (layers "F.Cu" "B.Cu") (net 11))
 (via (at 164.872899 74.586428) (size 0.6) (drill 0.3) (layers "F.Cu" "B.Cu") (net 11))
 (segment (start 166.985 124.81) (end 166.985 124.79) (width 0.2) (layer "B.Cu") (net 11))
 (segment (start 162.175 77.64) (end 164.872899 74.942101) (width 0.2) (layer "B.Cu") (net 11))
 (segment (start 166.985 124.79) (end 162.175 119.98) (width 0.2) (layer "B.Cu") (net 11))
 (segment (start 162.175 119.98) (end 162.175 77.64) (width 0.2) (layer "B.Cu") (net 11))
 (segment (start 164.872899 74.942101) (end 164.872899 74.586428) (width 0.2) (layer "B.Cu") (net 11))
 (segment (start 163.88 77.945) (end 163.875 77.94) (width 0.2) (layer "F.Cu") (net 4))
 (segment (start 166.335 68.32) (end 165.805 67.79) (width 0.2) (layer "F.Cu") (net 4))
 (segment (start 165.805 67.79) (end 160.335 67.79) (width 0.2) (layer "F.Cu") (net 4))
 (segment (start 166.355 68.32) (end 166.335 68.32) (width 0.2) (layer "F.Cu") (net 4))
 (segment (start 163.88 88.69) (end 163.88 77.945) (width 0.2) (layer "F.Cu") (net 4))
 (via (at 166.355 68.32) (size 0.6) (drill 0.3) (layers "F.Cu" "B.Cu") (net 4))
 (via (at 163.875 77.94) (size 0.6) (drill 0.3) (layers "F.Cu" "B.Cu") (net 4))
 (segment (start 166.354 76.068943) (end 166.354 75.7861) (width 0.2) (layer "B.Cu") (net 4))
 (segment (start 166.354 75.7861) (end 166.19145 75.62355) (width 0.2) (layer "B.Cu") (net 4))
 (segment (start 166.355 68.32) (end 166.355 74.6529) (width 0.2) (layer "B.Cu") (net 4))
 (segment (start 166.355 74.6529) (end 166.9211 75.219) (width 0.2) (layer "B.Cu") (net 4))
 (segment (start 167.203943 75.219) (end 167.556 75.571057) (width 0.2) (layer "B.Cu") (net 4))
 (segment (start 166.9211 75.219) (end 167.203943 75.219) (width 0.2) (layer "B.Cu") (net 4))
 (segment (start 167.556 75.571057) (end 167.556 76.068943) (width 0.2) (layer "B.Cu") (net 4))
 (segment (start 167.556 76.068943) (end 167.203943 76.421) (width 0.2) (layer "B.Cu") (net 4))
 (segment (start 166.706057 76.421) (end 166.354 76.068943) (width 0.2) (layer "B.Cu") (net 4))
 (segment (start 167.203943 76.421) (end 166.706057 76.421) (width 0.2) (layer "B.Cu") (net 4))
 (segment (start 166.19145 75.62355) (end 163.875 77.94) (width 0.2) (layer "B.Cu") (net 4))
 (segment (start 163.88 93.69) (end 163.88 99.035) (width 0.2) (layer "F.Cu") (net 5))
 (segment (start 165.045 100.2) (end 181.225 100.2) (width 0.2) (layer "F.Cu") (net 5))
 (segment (start 181.225 76.73) (end 180.315 75.82) (width 0.2) (layer "F.Cu") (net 5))
 (segment (start 164.725 70.26) (end 164.655 70.33) (width 0.2) (layer "F.Cu") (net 5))
 (segment (start 180.315 75.82) (end 166.955 75.82) (width 0.2) (layer "F.Cu") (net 5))
 (segment (start 164.655 70.33) (end 160.335 70.33) (width 0.2) (layer "F.Cu") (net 5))
 (segment (start 181.225 100.2) (end 181.225 76.73) (width 0.2) (layer "F.Cu") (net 5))
 (segment (start 165.085 70.26) (end 164.725 70.26) (width 0.2) (layer "F.Cu") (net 5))
 (segment (start 163.88 99.035) (end 165.045 100.2) (width 0.2) (layer "F.Cu") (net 5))
 (via (at 166.955 75.82) (size 0.6) (drill 0.3) (layers "F.Cu" "B.Cu") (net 5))
 (via (at 165.085 70.26) (size 0.6) (drill 0.3) (layers "F.Cu" "B.Cu") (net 5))
 (segment (start 165.575 70.75) (end 165.085 70.26) (width 0.2) (layer "B.Cu") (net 5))
 (segment (start 165.575 74.44) (end 165.575 70.75) (width 0.2) (layer "B.Cu") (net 5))
 (segment (start 166.955 75.82) (end 165.575 74.44) (width 0.2) (layer "B.Cu") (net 5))
 (segment (start 178.045 62.46) (end 178.055 62.45) (width 0.2) (layer "F.Cu") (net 6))
 (segment (start 162.579 99.584) (end 162.579 92.491) (width 0.2) (layer "F.Cu") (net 6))
 (segment (start 178.045 62.57) (end 178.045 62.46) (width 0.2) (layer "F.Cu") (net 6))
 (segment (start 181.815 101.22) (end 164.215 101.22) (width 0.2) (layer "F.Cu") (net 6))
 (segment (start 162.579 92.491) (end 163.88 91.19) (width 0.2) (layer "F.Cu") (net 6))
 (segment (start 171.035 62.57) (end 170.905 62.7) (width 0.2) (layer "F.Cu") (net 6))
 (segment (start 164.215 101.22) (end 162.579 99.584) (width 0.2) (layer "F.Cu") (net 6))
 (segment (start 178.055 62.45) (end 182.384 62.45) (width 0.2) (layer "F.Cu") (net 6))
 (segment (start 161.3295 62.71) (end 161.17 62.71) (width 0.2) (layer "F.Cu") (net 6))
 (segment (start 170.905 62.7) (end 163.595 62.7) (width 0.2) (layer "F.Cu") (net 6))
 (segment (start 182.384 100.651) (end 181.815 101.22) (width 0.2) (layer "F.Cu") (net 6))
 (segment (start 182.384 62.45) (end 182.384 100.651) (width 0.2) (layer "F.Cu") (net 6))
 (segment (start 161.4095 62.79) (end 161.3295 62.71) (width 0.2) (layer "F.Cu") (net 6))
 (segment (start 163.585 62.71) (end 160.335 62.71) (width 0.2) (layer "F.Cu") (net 6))
 (segment (start 163.595 62.7) (end 163.585 62.71) (width 0.2) (layer "F.Cu") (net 6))
 (via (at 178.045 62.57) (size 0.6) (drill 0.3) (layers "F.Cu" "B.Cu") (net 6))
 (via (at 171.035 62.57) (size 0.6) (drill 0.3) (layers "F.Cu" "B.Cu") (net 6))
 (segment (start 177.975 62.57) (end 177.955 62.55) (width 0.2) (layer "B.Cu") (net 6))
 (segment (start 177.955 62.55) (end 171.215 62.55) (width 0.2) (layer "B.Cu") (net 6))
 (segment (start 171.215 62.55) (end 171.195 62.57) (width 0.2) (layer "B.Cu") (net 6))
 (segment (start 178.045 62.57) (end 177.975 62.57) (width 0.2) (layer "B.Cu") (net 6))
 (segment (start 171.195 62.57) (end 171.035 62.57) (width 0.2) (layer "B.Cu") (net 6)))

